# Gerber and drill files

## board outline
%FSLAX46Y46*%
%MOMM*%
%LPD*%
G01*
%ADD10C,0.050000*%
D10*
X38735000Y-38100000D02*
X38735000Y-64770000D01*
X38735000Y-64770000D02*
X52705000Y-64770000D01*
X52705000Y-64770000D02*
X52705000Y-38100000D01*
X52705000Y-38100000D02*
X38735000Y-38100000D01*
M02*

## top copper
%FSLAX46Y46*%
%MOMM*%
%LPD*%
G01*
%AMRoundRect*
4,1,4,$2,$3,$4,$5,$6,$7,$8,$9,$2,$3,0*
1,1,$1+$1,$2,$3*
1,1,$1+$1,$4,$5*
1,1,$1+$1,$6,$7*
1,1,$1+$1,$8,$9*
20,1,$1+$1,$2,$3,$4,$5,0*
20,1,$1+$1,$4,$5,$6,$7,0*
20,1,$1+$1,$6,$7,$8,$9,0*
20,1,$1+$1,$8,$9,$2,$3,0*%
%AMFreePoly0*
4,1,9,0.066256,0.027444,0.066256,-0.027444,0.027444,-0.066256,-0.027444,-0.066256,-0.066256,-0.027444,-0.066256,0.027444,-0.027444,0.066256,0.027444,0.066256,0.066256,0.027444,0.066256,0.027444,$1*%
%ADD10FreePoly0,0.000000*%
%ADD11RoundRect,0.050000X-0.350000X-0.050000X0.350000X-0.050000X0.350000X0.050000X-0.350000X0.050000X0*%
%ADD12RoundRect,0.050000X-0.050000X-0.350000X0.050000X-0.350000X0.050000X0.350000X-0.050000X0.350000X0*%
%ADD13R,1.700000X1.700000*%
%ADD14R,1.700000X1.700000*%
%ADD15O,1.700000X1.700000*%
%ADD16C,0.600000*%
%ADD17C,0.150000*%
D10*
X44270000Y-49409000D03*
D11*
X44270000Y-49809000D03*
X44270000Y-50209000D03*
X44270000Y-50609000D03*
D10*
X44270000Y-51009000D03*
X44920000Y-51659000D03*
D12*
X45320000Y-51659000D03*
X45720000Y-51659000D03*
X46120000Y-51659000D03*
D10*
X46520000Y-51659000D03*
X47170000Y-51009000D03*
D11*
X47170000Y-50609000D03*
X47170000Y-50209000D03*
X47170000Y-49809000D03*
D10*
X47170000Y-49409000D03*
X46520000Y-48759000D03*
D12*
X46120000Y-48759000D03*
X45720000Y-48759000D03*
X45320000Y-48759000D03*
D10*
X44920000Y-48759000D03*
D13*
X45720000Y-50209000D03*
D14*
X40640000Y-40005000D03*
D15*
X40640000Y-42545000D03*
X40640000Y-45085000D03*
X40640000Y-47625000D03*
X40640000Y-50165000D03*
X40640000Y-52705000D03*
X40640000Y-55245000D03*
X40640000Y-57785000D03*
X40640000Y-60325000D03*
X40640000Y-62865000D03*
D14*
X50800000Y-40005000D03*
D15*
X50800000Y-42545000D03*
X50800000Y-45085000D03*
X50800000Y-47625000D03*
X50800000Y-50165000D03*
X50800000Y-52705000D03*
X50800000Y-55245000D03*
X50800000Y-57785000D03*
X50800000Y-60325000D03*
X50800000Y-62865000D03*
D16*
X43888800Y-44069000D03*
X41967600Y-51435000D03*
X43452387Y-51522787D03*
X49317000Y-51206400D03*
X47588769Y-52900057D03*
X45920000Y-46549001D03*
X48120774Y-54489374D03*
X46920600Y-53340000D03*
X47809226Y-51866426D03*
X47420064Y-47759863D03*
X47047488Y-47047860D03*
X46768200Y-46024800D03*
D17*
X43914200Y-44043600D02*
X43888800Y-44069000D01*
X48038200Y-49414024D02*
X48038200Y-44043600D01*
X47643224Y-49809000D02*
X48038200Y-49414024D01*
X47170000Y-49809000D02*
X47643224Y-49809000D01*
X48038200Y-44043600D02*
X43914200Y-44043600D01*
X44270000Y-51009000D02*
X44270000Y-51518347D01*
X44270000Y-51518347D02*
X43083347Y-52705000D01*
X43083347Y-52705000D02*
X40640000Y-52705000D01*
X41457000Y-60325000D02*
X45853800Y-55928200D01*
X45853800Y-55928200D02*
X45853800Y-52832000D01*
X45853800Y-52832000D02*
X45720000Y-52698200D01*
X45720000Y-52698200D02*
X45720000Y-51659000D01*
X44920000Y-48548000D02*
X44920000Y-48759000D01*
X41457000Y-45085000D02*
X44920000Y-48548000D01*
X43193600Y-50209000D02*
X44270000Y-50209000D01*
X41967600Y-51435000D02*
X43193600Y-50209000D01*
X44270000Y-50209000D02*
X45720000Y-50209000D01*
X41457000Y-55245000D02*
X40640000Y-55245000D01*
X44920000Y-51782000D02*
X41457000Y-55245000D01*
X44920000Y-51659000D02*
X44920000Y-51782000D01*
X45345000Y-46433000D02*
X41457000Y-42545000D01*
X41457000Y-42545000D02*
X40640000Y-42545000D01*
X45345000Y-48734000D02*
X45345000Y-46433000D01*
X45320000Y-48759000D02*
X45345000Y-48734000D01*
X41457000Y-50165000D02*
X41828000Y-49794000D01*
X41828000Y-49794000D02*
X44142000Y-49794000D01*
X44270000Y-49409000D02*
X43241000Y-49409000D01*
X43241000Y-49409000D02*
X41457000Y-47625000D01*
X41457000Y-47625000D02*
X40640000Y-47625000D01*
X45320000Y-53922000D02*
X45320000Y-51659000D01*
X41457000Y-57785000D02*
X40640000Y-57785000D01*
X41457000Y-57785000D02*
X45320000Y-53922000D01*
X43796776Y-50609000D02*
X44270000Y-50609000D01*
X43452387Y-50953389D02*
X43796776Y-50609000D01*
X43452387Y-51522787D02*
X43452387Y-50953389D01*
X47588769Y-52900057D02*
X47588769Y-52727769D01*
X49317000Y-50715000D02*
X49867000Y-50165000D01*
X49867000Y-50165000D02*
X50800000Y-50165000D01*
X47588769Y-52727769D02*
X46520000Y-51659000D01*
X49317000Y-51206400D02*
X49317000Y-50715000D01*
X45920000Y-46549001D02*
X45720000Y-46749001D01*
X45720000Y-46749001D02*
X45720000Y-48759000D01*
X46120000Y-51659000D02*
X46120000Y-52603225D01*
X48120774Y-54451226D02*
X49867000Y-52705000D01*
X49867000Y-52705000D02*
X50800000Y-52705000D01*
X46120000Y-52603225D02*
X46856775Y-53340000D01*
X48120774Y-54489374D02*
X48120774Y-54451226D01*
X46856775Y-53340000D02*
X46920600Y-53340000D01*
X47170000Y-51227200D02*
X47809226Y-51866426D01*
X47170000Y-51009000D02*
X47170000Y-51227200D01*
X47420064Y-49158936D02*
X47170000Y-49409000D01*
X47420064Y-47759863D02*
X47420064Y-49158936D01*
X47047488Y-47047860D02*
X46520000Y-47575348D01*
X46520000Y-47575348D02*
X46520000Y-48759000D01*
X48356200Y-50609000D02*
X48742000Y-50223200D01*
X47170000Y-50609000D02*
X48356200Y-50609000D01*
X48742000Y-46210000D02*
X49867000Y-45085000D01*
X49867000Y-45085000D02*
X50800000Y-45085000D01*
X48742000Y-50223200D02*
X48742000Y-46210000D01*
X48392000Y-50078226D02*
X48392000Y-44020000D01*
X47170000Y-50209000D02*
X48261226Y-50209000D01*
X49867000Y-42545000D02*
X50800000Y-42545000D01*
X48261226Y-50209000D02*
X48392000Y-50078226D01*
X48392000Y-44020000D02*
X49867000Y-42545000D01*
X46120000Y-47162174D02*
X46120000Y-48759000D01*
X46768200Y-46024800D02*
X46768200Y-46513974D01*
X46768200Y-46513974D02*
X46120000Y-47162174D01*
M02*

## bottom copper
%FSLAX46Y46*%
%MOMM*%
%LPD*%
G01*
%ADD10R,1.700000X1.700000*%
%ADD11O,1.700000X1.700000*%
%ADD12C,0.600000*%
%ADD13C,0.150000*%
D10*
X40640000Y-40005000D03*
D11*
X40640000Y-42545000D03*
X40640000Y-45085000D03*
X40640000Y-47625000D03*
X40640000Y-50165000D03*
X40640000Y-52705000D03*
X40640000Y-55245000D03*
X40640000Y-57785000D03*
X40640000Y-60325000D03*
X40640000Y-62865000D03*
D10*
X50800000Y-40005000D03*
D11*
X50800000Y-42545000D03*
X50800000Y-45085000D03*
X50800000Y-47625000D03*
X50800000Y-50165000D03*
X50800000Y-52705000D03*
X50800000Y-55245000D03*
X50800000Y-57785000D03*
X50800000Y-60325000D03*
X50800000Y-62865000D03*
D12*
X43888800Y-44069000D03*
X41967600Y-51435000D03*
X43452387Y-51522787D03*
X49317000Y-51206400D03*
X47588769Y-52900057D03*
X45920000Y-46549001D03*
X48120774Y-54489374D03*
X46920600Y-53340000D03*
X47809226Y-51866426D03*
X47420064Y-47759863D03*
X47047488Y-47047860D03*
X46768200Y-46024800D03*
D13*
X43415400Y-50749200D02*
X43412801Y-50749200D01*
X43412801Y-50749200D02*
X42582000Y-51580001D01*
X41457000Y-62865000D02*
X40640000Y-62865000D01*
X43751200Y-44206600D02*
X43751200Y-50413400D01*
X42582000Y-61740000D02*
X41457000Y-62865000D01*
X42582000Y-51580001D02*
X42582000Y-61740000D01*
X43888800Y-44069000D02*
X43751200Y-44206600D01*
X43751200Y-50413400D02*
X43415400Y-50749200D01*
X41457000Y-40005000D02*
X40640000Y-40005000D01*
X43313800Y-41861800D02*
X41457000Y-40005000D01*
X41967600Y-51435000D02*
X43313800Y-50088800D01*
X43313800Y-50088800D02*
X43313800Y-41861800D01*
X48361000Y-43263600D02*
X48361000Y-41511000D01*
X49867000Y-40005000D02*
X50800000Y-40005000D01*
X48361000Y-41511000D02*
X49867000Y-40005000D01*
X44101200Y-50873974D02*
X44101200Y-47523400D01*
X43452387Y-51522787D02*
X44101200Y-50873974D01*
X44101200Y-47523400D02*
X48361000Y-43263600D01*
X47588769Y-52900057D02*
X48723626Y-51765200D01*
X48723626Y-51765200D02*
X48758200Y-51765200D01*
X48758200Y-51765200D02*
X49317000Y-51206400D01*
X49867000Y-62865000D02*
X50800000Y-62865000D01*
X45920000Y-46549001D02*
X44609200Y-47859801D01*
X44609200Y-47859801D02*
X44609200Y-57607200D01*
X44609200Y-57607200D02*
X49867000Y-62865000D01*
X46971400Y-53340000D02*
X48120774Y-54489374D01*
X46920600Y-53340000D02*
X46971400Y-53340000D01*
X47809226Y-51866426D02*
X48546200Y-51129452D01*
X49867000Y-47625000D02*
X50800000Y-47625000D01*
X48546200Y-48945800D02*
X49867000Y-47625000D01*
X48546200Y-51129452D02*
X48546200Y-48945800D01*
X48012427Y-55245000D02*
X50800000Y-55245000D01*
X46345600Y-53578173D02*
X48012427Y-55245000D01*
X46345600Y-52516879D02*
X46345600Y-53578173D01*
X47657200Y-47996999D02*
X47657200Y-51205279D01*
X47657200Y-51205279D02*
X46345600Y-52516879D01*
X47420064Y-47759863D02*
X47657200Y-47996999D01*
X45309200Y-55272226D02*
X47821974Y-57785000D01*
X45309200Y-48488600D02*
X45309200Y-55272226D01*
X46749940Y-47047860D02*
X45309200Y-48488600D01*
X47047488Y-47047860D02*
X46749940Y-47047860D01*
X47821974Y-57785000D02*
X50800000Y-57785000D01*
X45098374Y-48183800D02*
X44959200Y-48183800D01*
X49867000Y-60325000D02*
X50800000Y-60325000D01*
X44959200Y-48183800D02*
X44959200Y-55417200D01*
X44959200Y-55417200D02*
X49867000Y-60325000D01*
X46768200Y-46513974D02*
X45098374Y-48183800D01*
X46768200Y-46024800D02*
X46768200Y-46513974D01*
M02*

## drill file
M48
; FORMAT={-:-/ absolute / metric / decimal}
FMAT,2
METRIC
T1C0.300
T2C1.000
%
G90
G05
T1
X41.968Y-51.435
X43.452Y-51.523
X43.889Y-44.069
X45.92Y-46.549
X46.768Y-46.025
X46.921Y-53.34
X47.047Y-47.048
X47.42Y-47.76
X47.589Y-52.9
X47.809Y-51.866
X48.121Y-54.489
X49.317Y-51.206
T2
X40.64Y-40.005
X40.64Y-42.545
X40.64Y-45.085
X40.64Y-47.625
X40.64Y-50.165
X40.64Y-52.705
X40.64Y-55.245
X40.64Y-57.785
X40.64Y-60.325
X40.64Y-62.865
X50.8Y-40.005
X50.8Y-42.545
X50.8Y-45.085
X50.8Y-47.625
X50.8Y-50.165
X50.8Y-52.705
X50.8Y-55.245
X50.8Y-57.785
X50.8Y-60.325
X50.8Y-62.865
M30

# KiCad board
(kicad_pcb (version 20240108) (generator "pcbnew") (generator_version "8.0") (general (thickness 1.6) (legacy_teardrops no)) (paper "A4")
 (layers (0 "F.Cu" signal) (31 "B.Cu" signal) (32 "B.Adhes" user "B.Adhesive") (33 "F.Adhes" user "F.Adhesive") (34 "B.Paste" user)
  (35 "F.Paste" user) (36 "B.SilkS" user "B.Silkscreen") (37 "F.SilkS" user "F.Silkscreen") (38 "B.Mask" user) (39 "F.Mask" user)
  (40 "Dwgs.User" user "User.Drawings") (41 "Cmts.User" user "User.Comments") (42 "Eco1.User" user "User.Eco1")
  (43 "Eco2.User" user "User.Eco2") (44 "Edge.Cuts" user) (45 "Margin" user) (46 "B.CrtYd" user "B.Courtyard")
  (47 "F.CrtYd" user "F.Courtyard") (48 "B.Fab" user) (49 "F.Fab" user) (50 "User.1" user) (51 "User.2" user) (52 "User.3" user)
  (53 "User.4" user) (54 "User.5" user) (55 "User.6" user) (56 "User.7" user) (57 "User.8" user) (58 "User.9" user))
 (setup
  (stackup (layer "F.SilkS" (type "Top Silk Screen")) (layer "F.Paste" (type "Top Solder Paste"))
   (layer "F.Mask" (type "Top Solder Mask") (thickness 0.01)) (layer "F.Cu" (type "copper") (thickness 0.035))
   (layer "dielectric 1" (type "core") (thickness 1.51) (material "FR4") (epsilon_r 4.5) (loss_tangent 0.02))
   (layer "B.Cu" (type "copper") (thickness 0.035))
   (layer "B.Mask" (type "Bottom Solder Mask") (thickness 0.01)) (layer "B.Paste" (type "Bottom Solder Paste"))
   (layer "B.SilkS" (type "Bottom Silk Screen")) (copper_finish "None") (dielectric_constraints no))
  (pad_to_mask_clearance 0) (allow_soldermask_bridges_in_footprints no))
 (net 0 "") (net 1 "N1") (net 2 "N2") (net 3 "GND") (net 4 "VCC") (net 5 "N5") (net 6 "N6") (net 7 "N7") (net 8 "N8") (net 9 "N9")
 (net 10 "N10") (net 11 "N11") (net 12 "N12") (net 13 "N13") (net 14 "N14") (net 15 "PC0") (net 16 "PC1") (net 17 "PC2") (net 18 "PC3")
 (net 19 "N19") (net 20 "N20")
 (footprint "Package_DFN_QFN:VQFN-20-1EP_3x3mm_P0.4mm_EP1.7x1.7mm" (layer "F.Cu") (at 45.72 50.209)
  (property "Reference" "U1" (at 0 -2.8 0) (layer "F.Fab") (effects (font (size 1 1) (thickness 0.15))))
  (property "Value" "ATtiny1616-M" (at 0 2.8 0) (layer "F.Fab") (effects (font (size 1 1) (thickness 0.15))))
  (pad "" smd roundrect (at -0.425 -0.425) (size 0.69 0.69) (layers "F.Paste") (roundrect_rratio 0.25))
  (pad "" smd roundrect (at -0.425 0.425) (size 0.69 0.69) (layers "F.Paste") (roundrect_rratio 0.25))
  (pad "" smd roundrect (at 0.425 -0.425) (size 0.69 0.69) (layers "F.Paste") (roundrect_rratio 0.25))
  (pad "" smd roundrect (at 0.425 0.425) (size 0.69 0.69) (layers "F.Paste") (roundrect_rratio 0.25))
  (pad "1" smd custom (at -1.45 -0.8) (size 0.143431 0.143431) (layers "F.Cu" "F.Paste" "F.Mask") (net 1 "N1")
   (options (clearance outline) (anchor circle)) (primitives))
  (pad "2" smd roundrect (at -1.45 -0.4) (size 0.8 0.2) (layers "F.Cu" "F.Paste" "F.Mask") (roundrect_rratio 0.25) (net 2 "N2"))
  (pad "3" smd roundrect (at -1.45 0) (size 0.8 0.2) (layers "F.Cu" "F.Paste" "F.Mask") (roundrect_rratio 0.25) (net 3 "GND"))
  (pad "4" smd roundrect (at -1.45 0.4) (size 0.8 0.2) (layers "F.Cu" "F.Paste" "F.Mask") (roundrect_rratio 0.25) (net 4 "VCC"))
  (pad "5" smd custom (at -1.45 0.8) (size 0.143431 0.143431) (layers "F.Cu" "F.Paste" "F.Mask") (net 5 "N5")
   (options (clearance outline) (anchor circle)) (primitives))
  (pad "6" smd custom (at -0.8 1.45) (size 0.143431 0.143431) (layers "F.Cu" "F.Paste" "F.Mask") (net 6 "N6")
   (options (clearance outline) (anchor circle)) (primitives))
  (pad "7" smd roundrect (at -0.4 1.45) (size 0.2 0.8) (layers "F.Cu" "F.Paste" "F.Mask") (roundrect_rratio 0.25) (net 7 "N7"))
  (pad "8" smd roundrect (at 0 1.45) (size 0.2 0.8) (layers "F.Cu" "F.Paste" "F.Mask") (roundrect_rratio 0.25) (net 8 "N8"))
  (pad "9" smd roundrect (at 0.4 1.45) (size 0.2 0.8) (layers "F.Cu" "F.Paste" "F.Mask") (roundrect_rratio 0.25) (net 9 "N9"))
  (pad "10" smd custom (at 0.8 1.45) (size 0.143431 0.143431) (layers "F.Cu" "F.Paste" "F.Mask") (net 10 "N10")
   (options (clearance outline) (anchor circle)) (primitives))
  (pad "11" smd custom (at 1.45 0.8) (size 0.143431 0.143431) (layers "F.Cu" "F.Paste" "F.Mask") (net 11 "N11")
   (options (clearance outline) (anchor circle)) (primitives))
  (pad "12" smd roundrect (at 1.45 0.4) (size 0.8 0.2) (layers "F.Cu" "F.Paste" "F.Mask") (roundrect_rratio 0.25) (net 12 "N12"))
  (pad "13" smd roundrect (at 1.45 0) (size 0.8 0.2) (layers "F.Cu" "F.Paste" "F.Mask") (roundrect_rratio 0.25) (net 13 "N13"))
  (pad "14" smd roundrect (at 1.45 -0.4) (size 0.8 0.2) (layers "F.Cu" "F.Paste" "F.Mask") (roundrect_rratio 0.25) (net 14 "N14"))
  (pad "15" smd custom (at 1.45 -0.8) (size 0.143431 0.143431) (layers "F.Cu" "F.Paste" "F.Mask") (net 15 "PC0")
   (options (clearance outline) (anchor circle)) (primitives))
  (pad "16" smd custom (at 0.8 -1.45) (size 0.143431 0.143431) (layers "F.Cu" "F.Paste" "F.Mask") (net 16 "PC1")
   (options (clearance outline) (anchor circle)) (primitives))
  (pad "17" smd roundrect (at 0.4 -1.45) (size 0.2 0.8) (layers "F.Cu" "F.Paste" "F.Mask") (roundrect_rratio 0.25) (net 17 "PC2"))
  (pad "18" smd roundrect (at 0 -1.45) (size 0.2 0.8) (layers "F.Cu" "F.Paste" "F.Mask") (roundrect_rratio 0.25) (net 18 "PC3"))
  (pad "19" smd roundrect (at -0.4 -1.45) (size 0.2 0.8) (layers "F.Cu" "F.Paste" "F.Mask") (roundrect_rratio 0.25) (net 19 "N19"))
  (pad "20" smd custom (at -0.8 -1.45) (size 0.143431 0.143431) (layers "F.Cu" "F.Paste" "F.Mask") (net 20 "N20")
   (options (clearance outline) (anchor circle)) (primitives))
  (pad "21" smd rect (at 0 0) (size 1.7 1.7) (layers "F.Cu" "F.Mask") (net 3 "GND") (zone_connect 2)))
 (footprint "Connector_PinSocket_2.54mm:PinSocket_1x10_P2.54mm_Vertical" (layer "B.Cu") (at 40.64 40.005 180)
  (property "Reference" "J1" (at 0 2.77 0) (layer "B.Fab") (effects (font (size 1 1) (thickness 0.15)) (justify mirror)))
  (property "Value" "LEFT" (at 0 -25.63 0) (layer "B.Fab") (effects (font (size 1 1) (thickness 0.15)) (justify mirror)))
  (pad "1" thru_hole rect (at 0 0 180) (size 1.7 1.7) (drill 1) (layers "*.Cu" "*.Mask") (remove_unused_layers no) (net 3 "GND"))
  (pad "2" thru_hole oval (at 0 -2.54 180) (size 1.7 1.7) (drill 1) (layers "*.Cu" "*.Mask") (remove_unused_layers no) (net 19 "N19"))
  (pad "3" thru_hole oval (at 0 -5.08 180) (size 1.7 1.7) (drill 1) (layers "*.Cu" "*.Mask") (remove_unused_layers no) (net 20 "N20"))
  (pad "4" thru_hole oval (at 0 -7.62 180) (size 1.7 1.7) (drill 1) (layers "*.Cu" "*.Mask") (remove_unused_layers no) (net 1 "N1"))
  (pad "5" thru_hole oval (at 0 -10.16 180) (size 1.7 1.7) (drill 1) (layers "*.Cu" "*.Mask") (remove_unused_layers no) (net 2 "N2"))
  (pad "6" thru_hole oval (at 0 -12.7 180) (size 1.7 1.7) (drill 1) (layers "*.Cu" "*.Mask") (remove_unused_layers no) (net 5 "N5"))
  (pad "7" thru_hole oval (at 0 -15.24 180) (size 1.7 1.7) (drill 1) (layers "*.Cu" "*.Mask") (remove_unused_layers no) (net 6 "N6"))
  (pad "8" thru_hole oval (at 0 -17.78 180) (size 1.7 1.7) (drill 1) (layers "*.Cu" "*.Mask") (remove_unused_layers no) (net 7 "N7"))
  (pad "9" thru_hole oval (at 0 -20.32 180) (size 1.7 1.7) (drill 1) (layers "*.Cu" "*.Mask") (remove_unused_layers no) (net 8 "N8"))
  (pad "10" thru_hole oval (at 0 -22.86 180) (size 1.7 1.7) (drill 1) (layers "*.Cu" "*.Mask") (remove_unused_layers no) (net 14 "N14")))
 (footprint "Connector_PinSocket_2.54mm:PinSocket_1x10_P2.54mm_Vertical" (layer "B.Cu") (at 50.8 40.005 180)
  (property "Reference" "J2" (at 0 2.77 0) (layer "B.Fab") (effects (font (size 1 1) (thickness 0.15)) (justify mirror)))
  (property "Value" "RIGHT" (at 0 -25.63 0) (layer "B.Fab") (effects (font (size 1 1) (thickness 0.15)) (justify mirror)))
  (pad "1" thru_hole rect (at 0 0 180) (size 1.7 1.7) (drill 1) (layers "*.Cu" "*.Mask") (remove_unused_layers no) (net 4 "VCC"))
  (pad "2" thru_hole oval (at 0 -2.54 180) (size 1.7 1.7) (drill 1) (layers "*.Cu" "*.Mask") (remove_unused_layers no) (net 13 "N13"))
  (pad "3" thru_hole oval (at 0 -5.08 180) (size 1.7 1.7) (drill 1) (layers "*.Cu" "*.Mask") (remove_unused_layers no) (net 12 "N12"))
  (pad "4" thru_hole oval (at 0 -7.62 180) (size 1.7 1.7) (drill 1) (layers "*.Cu" "*.Mask") (remove_unused_layers no) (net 11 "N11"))
  (pad "5" thru_hole oval (at 0 -10.16 180) (size 1.7 1.7) (drill 1) (layers "*.Cu" "*.Mask") (remove_unused_layers no) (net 10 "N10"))
  (pad "6" thru_hole oval (at 0 -12.7 180) (size 1.7 1.7) (drill 1) (layers "*.Cu" "*.Mask") (remove_unused_layers no) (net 9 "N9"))
  (pad "7" thru_hole oval (at 0 -15.24 180) (size 1.7 1.7) (drill 1) (layers "*.Cu" "*.Mask") (remove_unused_layers no) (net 15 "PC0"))
  (pad "8" thru_hole oval (at 0 -17.78 180) (size 1.7 1.7) (drill 1) (layers "*.Cu" "*.Mask") (remove_unused_layers no) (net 16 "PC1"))
  (pad "9" thru_hole oval (at 0 -20.32 180) (size 1.7 1.7) (drill 1) (layers "*.Cu" "*.Mask") (remove_unused_layers no) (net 17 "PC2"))
  (pad "10" thru_hole oval (at 0 -22.86 180) (size 1.7 1.7) (drill 1) (layers "*.Cu" "*.Mask") (remove_unused_layers no) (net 18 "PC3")))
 (gr_line (start 38.735 38.1) (end 38.735 64.77) (stroke (width 0.05) (type default)) (layer "Edge.Cuts"))
 (gr_line (start 38.735 64.77) (end 52.705 64.77) (stroke (width 0.05) (type default)) (layer "Edge.Cuts"))
 (gr_line (start 52.705 64.77) (end 52.705 38.1) (stroke (width 0.05) (type default)) (layer "Edge.Cuts"))
 (gr_line (start 52.705 38.1) (end 38.735 38.1) (stroke (width 0.05) (type default)) (layer "Edge.Cuts"))
 (segment (start 43.9142 44.0436) (end 43.8888 44.069) (width 0.15) (layer "F.Cu") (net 14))
 (segment (start 48.0382 49.414024) (end 48.0382 44.0436) (width 0.15) (layer "F.Cu") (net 14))
 (segment (start 47.643224 49.809) (end 48.0382 49.414024) (width 0.15) (layer "F.Cu") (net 14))
 (segment (start 47.17 49.809) (end 47.643224 49.809) (width 0.15) (layer "F.Cu") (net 14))
 (segment (start 48.0382 44.0436) (end 43.9142 44.0436) (width 0.15) (layer "F.Cu") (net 14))
 (via (at 43.8888 44.069) (size 0.6) (drill 0.3) (layers "F.Cu" "B.Cu") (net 14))
 (segment (start 43.4154 50.7492) (end 43.412801 50.7492) (width 0.15) (layer "B.Cu") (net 14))
 (segment (start 43.412801 50.7492) (end 42.582 51.580001) (width 0.15) (layer "B.Cu") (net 14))
 (segment (start 41.457 62.865) (end 40.64 62.865) (width 0.15) (layer "B.Cu") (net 14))
 (segment (start 43.7512 44.2066) (end 43.7512 50.4134) (width 0.15) (layer "B.Cu") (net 14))
 (segment (start 42.582 61.74) (end 41.457 62.865) (width 0.15) (layer "B.Cu") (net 14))
 (segment (start 42.582 51.580001) (end 42.582 61.74) (width 0.15) (layer "B.Cu") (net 14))
 (segment (start 43.8888 44.069) (end 43.7512 44.2066) (width 0.15) (layer "B.Cu") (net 14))
 (segment (start 43.7512 50.4134) (end 43.4154 50.7492) (width 0.15) (layer "B.Cu") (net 14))
 (segment (start 44.27 51.009) (end 44.27 51.518347) (width 0.15) (layer "F.Cu") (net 5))
 (segment (start 44.27 51.518347) (end 43.083347 52.705) (width 0.15) (layer "F.Cu") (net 5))
 (segment (start 43.083347 52.705) (end 40.64 52.705) (width 0.15) (layer "F.Cu") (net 5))
 (segment (start 41.457 60.325) (end 45.8538 55.9282) (width 0.15) (layer "F.Cu") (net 8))
 (segment (start 45.8538 55.9282) (end 45.8538 52.832) (width 0.15) (layer "F.Cu") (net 8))
 (segment (start 45.8538 52.832) (end 45.72 52.6982) (width 0.15) (layer "F.Cu") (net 8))
 (segment (start 45.72 52.6982) (end 45.72 51.659) (width 0.15) (layer "F.Cu") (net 8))
 (segment (start 44.92 48.548) (end 44.92 48.759) (width 0.15) (layer "F.Cu") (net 20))
 (segment (start 41.457 45.085) (end 44.92 48.548) (width 0.15) (layer "F.Cu") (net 20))
 (segment (start 43.1936 50.209) (end 44.27 50.209) (width 0.15) (layer "F.Cu") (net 3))
 (segment (start 41.9676 51.435) (end 43.1936 50.209) (width 0.15) (layer "F.Cu") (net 3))
 (segment (start 44.27 50.209) (end 45.72 50.209) (width 0.15) (layer "F.Cu") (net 3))
 (via (at 41.9676 51.435) (size 0.6) (drill 0.3) (layers "F.Cu" "B.Cu") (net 3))
 (segment (start 41.457 40.005) (end 40.64 40.005) (width 0.15) (layer "B.Cu") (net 3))
 (segment (start 43.3138 41.8618) (end 41.457 40.005) (width 0.15) (layer "B.Cu") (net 3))
 (segment (start 41.9676 51.435) (end 43.3138 50.0888) (width 0.15) (layer "B.Cu") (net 3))
 (segment (start 43.3138 50.0888) (end 43.3138 41.8618) (width 0.15) (layer "B.Cu") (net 3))
 (segment (start 41.457 55.245) (end 40.64 55.245) (width 0.15) (layer "F.Cu") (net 6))
 (segment (start 44.92 51.782) (end 41.457 55.245) (width 0.15) (layer "F.Cu") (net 6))
 (segment (start 44.92 51.659) (end 44.92 51.782) (width 0.15) (layer "F.Cu") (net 6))
 (segment (start 45.345 46.433) (end 41.457 42.545) (width 0.15) (layer "F.Cu") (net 19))
 (segment (start 41.457 42.545) (end 40.64 42.545) (width 0.15) (layer "F.Cu") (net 19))
 (segment (start 45.345 48.734) (end 45.345 46.433) (width 0.15) (layer "F.Cu") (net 19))
 (segment (start 45.32 48.759) (end 45.345 48.734) (width 0.15) (layer "F.Cu") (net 19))
 (segment (start 41.457 50.165) (end 41.828 49.794) (width 0.15) (layer "F.Cu") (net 2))
 (segment (start 41.828 49.794) (end 44.142 49.794) (width 0.15) (layer "F.Cu") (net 2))
 (segment (start 44.27 49.409) (end 43.241 49.409) (width 0.15) (layer "F.Cu") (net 1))
 (segment (start 43.241 49.409) (end 41.457 47.625) (width 0.15) (layer "F.Cu") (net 1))
 (segment (start 41.457 47.625) (end 40.64 47.625) (width 0.15) (layer "F.Cu") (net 1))
 (segment (start 45.32 53.922) (end 45.32 51.659) (width 0.15) (layer "F.Cu") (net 7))
 (segment (start 41.457 57.785) (end 40.64 57.785) (width 0.15) (layer "F.Cu") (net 7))
 (segment (start 41.457 57.785) (end 45.32 53.922) (width 0.15) (layer "F.Cu") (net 7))
 (segment (start 43.796776 50.609) (end 44.27 50.609) (width 0.15) (layer "F.Cu") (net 4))
 (segment (start 43.452387 50.953389) (end 43.796776 50.609) (width 0.15) (layer "F.Cu") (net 4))
 (segment (start 43.452387 51.522787) (end 43.452387 50.953389) (width 0.15) (layer "F.Cu") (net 4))
 (via (at 43.452387 51.522787) (size 0.6) (drill 0.3) (layers "F.Cu" "B.Cu") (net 4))
 (segment (start 48.361 43.2636) (end 48.361 41.511) (width 0.15) (layer "B.Cu") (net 4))
 (segment (start 49.867 40.005) (end 50.8 40.005) (width 0.15) (layer "B.Cu") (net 4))
 (segment (start 48.361 41.511) (end 49.867 40.005) (width 0.15) (layer "B.Cu") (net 4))
 (segment (start 44.1012 50.873974) (end 44.1012 47.5234) (width 0.15) (layer "B.Cu") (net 4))
 (segment (start 43.452387 51.522787) (end 44.1012 50.873974) (width 0.15) (layer "B.Cu") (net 4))
 (segment (start 44.1012 47.5234) (end 48.361 43.2636) (width 0.15) (layer "B.Cu") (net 4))
 (segment (start 47.588769 52.900057) (end 47.588769 52.727769) (width 0.15) (layer "F.Cu") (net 10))
 (segment (start 49.317 50.715) (end 49.867 50.165) (width 0.15) (layer "F.Cu") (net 10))
 (segment (start 49.867 50.165) (end 50.8 50.165) (width 0.15) (layer "F.Cu") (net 10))
 (segment (start 47.588769 52.727769) (end 46.52 51.659) (width 0.15) (layer "F.Cu") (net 10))
 (segment (start 49.317 51.2064) (end 49.317 50.715) (width 0.15) (layer "F.Cu") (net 10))
 (via (at 49.317 51.2064) (size 0.6) (drill 0.3) (layers "F.Cu" "B.Cu") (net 10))
 (via (at 47.588769 52.900057) (size 0.6) (drill 0.3) (layers "F.Cu" "B.Cu") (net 10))
 (segment (start 47.588769 52.900057) (end 48.723626 51.7652) (width 0.15) (layer "B.Cu") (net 10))
 (segment (start 48.723626 51.7652) (end 48.7582 51.7652) (width 0.15) (layer "B.Cu") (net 10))
 (segment (start 48.7582 51.7652) (end 49.317 51.2064) (width 0.15) (layer "B.Cu") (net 10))
 (segment (start 45.92 46.549001) (end 45.72 46.749001) (width 0.15) (layer "F.Cu") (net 18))
 (segment (start 45.72 46.749001) (end 45.72 48.759) (width 0.15) (layer "F.Cu") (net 18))
 (via (at 45.92 46.549001) (size 0.6) (drill 0.3) (layers "F.Cu" "B.Cu") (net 18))
 (segment (start 49.867 62.865) (end 50.8 62.865) (width 0.15) (layer "B.Cu") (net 18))
 (segment (start 45.92 46.549001) (end 44.6092 47.859801) (width 0.15) (layer "B.Cu") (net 18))
 (segment (start 44.6092 47.859801) (end 44.6092 57.6072) (width 0.15) (layer "B.Cu") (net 18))
 (segment (start 44.6092 57.6072) (end 49.867 62.865) (width 0.15) (layer "B.Cu") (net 18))
 (segment (start 46.12 51.659) (end 46.12 52.603225) (width 0.15) (layer "F.Cu") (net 9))
 (segment (start 48.120774 54.451226) (end 49.867 52.705) (width 0.15) (layer "F.Cu") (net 9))
 (segment (start 49.867 52.705) (end 50.8 52.705) (width 0.15) (layer "F.Cu") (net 9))
 (segment (start 46.12 52.603225) (end 46.856775 53.34) (width 0.15) (layer "F.Cu") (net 9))
 (segment (start 48.120774 54.489374) (end 48.120774 54.451226) (width 0.15) (layer "F.Cu") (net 9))
 (segment (start 46.856775 53.34) (end 46.9206 53.34) (width 0.15) (layer "F.Cu") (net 9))
 (via (at 48.120774 54.489374) (size 0.6) (drill 0.3) (layers "F.Cu" "B.Cu") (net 9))
 (via (at 46.9206 53.34) (size 0.6) (drill 0.3) (layers "F.Cu" "B.Cu") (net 9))
 (segment (start 46.9714 53.34) (end 48.120774 54.489374) (width 0.15) (layer "B.Cu") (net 9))
 (segment (start 46.9206 53.34) (end 46.9714 53.34) (width 0.15) (layer "B.Cu") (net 9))
 (segment (start 47.17 51.2272) (end 47.809226 51.866426) (width 0.15) (layer "F.Cu") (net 11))
 (segment (start 47.17 51.009) (end 47.17 51.2272) (width 0.15) (layer "F.Cu") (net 11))
 (via (at 47.809226 51.866426) (size 0.6) (drill 0.3) (layers "F.Cu" "B.Cu") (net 11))
 (segment (start 47.809226 51.866426) (end 48.5462 51.129452) (width 0.15) (layer "B.Cu") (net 11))
 (segment (start 49.867 47.625) (end 50.8 47.625) (width 0.15) (layer "B.Cu") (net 11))
 (segment (start 48.5462 48.9458) (end 49.867 47.625) (width 0.15) (layer "B.Cu") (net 11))
 (segment (start 48.5462 51.129452) (end 48.5462 48.9458) (width 0.15) (layer "B.Cu") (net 11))
 (segment (start 47.420064 49.158936) (end 47.17 49.409) (width 0.15) (layer "F.Cu") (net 15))
 (segment (start 47.420064 47.759863) (end 47.420064 49.158936) (width 0.15) (layer "F.Cu") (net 15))
 (via (at 47.420064 47.759863) (size 0.6) (drill 0.3) (layers "F.Cu" "B.Cu") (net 15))
 (segment (start 48.012427 55.245) (end 50.8 55.245) (width 0.15) (layer "B.Cu") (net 15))
 (segment (start 46.3456 53.578173) (end 48.012427 55.245) (width 0.15) (layer "B.Cu") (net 15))
 (segment (start 46.3456 52.516879) (end 46.3456 53.578173) (width 0.15) (layer "B.Cu") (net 15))
 (segment (start 47.6572 47.996999) (end 47.6572 51.205279) (width 0.15) (layer "B.Cu") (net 15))
 (segment (start 47.6572 51.205279) (end 46.3456 52.516879) (width 0.15) (layer "B.Cu") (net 15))
 (segment (start 47.420064 47.759863) (end 47.6572 47.996999) (width 0.15) (layer "B.Cu") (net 15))
 (segment (start 47.047488 47.04786) (end 46.52 47.575348) (width 0.15) (layer "F.Cu") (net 16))
 (segment (start 46.52 47.575348) (end 46.52 48.759) (width 0.15) (layer "F.Cu") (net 16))
 (via (at 47.047488 47.04786) (size 0.6) (drill 0.3) (layers "F.Cu" "B.Cu") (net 16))
 (segment (start 45.3092 55.272226) (end 47.821974 57.785) (width 0.15) (layer "B.Cu") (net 16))
 (segment (start 45.3092 48.4886) (end 45.3092 55.272226) (width 0.15) (layer "B.Cu") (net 16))
 (segment (start 46.74994 47.04786) (end 45.3092 48.4886) (width 0.15) (layer "B.Cu") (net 16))
 (segment (start 47.047488 47.04786) (end 46.74994 47.04786) (width 0.15) (layer "B.Cu") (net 16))
 (segment (start 47.821974 57.785) (end 50.8 57.785) (width 0.15) (layer "B.Cu") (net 16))
 (segment (start 48.3562 50.609) (end 48.742 50.2232) (width 0.15) (layer "F.Cu") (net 12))
 (segment (start 47.17 50.609) (end 48.3562 50.609) (width 0.15) (layer "F.Cu") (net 12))
 (segment (start 48.742 46.21) (end 49.867 45.085) (width 0.15) (layer "F.Cu") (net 12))
 (segment (start 49.867 45.085) (end 50.8 45.085) (width 0.15) (layer "F.Cu") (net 12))
 (segment (start 48.742 50.2232) (end 48.742 46.21) (width 0.15) (layer "F.Cu") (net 12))
 (segment (start 48.392 50.078226) (end 48.392 44.02) (width 0.15) (layer "F.Cu") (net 13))
 (segment (start 47.17 50.209) (end 48.261226 50.209) (width 0.15) (layer "F.Cu") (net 13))
 (segment (start 49.867 42.545) (end 50.8 42.545) (width 0.15) (layer "F.Cu") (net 13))
 (segment (start 48.261226 50.209) (end 48.392 50.078226) (width 0.15) (layer "F.Cu") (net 13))
 (segment (start 48.392 44.02) (end 49.867 42.545) (width 0.15) (layer "F.Cu") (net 13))
 (segment (start 46.12 47.162174) (end 46.12 48.759) (width 0.15) (layer "F.Cu") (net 17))
 (segment (start 46.7682 46.0248) (end 46.7682 46.513974) (width 0.15) (layer "F.Cu") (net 17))
 (segment (start 46.7682 46.513974) (end 46.12 47.162174) (width 0.15) (layer "F.Cu") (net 17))
 (via (at 46.7682 46.0248) (size 0.6) (drill 0.3) (layers "F.Cu" "B.Cu") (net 17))
 (segment (start 45.098374 48.1838) (end 44.9592 48.1838) (width 0.15) (layer "B.Cu") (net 17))
 (segment (start 49.867 60.325) (end 50.8 60.325) (width 0.15) (layer "B.Cu") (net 17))
 (segment (start 44.9592 48.1838) (end 44.9592 55.4172) (width 0.15) (layer "B.Cu") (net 17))
 (segment (start 44.9592 55.4172) (end 49.867 60.325) (width 0.15) (layer "B.Cu") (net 17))
 (segment (start 46.7682 46.513974) (end 45.098374 48.1838) (width 0.15) (layer "B.Cu") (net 17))
 (segment (start 46.7682 46.0248) (end 46.7682 46.513974) (width 0.15) (layer "B.Cu") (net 17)))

